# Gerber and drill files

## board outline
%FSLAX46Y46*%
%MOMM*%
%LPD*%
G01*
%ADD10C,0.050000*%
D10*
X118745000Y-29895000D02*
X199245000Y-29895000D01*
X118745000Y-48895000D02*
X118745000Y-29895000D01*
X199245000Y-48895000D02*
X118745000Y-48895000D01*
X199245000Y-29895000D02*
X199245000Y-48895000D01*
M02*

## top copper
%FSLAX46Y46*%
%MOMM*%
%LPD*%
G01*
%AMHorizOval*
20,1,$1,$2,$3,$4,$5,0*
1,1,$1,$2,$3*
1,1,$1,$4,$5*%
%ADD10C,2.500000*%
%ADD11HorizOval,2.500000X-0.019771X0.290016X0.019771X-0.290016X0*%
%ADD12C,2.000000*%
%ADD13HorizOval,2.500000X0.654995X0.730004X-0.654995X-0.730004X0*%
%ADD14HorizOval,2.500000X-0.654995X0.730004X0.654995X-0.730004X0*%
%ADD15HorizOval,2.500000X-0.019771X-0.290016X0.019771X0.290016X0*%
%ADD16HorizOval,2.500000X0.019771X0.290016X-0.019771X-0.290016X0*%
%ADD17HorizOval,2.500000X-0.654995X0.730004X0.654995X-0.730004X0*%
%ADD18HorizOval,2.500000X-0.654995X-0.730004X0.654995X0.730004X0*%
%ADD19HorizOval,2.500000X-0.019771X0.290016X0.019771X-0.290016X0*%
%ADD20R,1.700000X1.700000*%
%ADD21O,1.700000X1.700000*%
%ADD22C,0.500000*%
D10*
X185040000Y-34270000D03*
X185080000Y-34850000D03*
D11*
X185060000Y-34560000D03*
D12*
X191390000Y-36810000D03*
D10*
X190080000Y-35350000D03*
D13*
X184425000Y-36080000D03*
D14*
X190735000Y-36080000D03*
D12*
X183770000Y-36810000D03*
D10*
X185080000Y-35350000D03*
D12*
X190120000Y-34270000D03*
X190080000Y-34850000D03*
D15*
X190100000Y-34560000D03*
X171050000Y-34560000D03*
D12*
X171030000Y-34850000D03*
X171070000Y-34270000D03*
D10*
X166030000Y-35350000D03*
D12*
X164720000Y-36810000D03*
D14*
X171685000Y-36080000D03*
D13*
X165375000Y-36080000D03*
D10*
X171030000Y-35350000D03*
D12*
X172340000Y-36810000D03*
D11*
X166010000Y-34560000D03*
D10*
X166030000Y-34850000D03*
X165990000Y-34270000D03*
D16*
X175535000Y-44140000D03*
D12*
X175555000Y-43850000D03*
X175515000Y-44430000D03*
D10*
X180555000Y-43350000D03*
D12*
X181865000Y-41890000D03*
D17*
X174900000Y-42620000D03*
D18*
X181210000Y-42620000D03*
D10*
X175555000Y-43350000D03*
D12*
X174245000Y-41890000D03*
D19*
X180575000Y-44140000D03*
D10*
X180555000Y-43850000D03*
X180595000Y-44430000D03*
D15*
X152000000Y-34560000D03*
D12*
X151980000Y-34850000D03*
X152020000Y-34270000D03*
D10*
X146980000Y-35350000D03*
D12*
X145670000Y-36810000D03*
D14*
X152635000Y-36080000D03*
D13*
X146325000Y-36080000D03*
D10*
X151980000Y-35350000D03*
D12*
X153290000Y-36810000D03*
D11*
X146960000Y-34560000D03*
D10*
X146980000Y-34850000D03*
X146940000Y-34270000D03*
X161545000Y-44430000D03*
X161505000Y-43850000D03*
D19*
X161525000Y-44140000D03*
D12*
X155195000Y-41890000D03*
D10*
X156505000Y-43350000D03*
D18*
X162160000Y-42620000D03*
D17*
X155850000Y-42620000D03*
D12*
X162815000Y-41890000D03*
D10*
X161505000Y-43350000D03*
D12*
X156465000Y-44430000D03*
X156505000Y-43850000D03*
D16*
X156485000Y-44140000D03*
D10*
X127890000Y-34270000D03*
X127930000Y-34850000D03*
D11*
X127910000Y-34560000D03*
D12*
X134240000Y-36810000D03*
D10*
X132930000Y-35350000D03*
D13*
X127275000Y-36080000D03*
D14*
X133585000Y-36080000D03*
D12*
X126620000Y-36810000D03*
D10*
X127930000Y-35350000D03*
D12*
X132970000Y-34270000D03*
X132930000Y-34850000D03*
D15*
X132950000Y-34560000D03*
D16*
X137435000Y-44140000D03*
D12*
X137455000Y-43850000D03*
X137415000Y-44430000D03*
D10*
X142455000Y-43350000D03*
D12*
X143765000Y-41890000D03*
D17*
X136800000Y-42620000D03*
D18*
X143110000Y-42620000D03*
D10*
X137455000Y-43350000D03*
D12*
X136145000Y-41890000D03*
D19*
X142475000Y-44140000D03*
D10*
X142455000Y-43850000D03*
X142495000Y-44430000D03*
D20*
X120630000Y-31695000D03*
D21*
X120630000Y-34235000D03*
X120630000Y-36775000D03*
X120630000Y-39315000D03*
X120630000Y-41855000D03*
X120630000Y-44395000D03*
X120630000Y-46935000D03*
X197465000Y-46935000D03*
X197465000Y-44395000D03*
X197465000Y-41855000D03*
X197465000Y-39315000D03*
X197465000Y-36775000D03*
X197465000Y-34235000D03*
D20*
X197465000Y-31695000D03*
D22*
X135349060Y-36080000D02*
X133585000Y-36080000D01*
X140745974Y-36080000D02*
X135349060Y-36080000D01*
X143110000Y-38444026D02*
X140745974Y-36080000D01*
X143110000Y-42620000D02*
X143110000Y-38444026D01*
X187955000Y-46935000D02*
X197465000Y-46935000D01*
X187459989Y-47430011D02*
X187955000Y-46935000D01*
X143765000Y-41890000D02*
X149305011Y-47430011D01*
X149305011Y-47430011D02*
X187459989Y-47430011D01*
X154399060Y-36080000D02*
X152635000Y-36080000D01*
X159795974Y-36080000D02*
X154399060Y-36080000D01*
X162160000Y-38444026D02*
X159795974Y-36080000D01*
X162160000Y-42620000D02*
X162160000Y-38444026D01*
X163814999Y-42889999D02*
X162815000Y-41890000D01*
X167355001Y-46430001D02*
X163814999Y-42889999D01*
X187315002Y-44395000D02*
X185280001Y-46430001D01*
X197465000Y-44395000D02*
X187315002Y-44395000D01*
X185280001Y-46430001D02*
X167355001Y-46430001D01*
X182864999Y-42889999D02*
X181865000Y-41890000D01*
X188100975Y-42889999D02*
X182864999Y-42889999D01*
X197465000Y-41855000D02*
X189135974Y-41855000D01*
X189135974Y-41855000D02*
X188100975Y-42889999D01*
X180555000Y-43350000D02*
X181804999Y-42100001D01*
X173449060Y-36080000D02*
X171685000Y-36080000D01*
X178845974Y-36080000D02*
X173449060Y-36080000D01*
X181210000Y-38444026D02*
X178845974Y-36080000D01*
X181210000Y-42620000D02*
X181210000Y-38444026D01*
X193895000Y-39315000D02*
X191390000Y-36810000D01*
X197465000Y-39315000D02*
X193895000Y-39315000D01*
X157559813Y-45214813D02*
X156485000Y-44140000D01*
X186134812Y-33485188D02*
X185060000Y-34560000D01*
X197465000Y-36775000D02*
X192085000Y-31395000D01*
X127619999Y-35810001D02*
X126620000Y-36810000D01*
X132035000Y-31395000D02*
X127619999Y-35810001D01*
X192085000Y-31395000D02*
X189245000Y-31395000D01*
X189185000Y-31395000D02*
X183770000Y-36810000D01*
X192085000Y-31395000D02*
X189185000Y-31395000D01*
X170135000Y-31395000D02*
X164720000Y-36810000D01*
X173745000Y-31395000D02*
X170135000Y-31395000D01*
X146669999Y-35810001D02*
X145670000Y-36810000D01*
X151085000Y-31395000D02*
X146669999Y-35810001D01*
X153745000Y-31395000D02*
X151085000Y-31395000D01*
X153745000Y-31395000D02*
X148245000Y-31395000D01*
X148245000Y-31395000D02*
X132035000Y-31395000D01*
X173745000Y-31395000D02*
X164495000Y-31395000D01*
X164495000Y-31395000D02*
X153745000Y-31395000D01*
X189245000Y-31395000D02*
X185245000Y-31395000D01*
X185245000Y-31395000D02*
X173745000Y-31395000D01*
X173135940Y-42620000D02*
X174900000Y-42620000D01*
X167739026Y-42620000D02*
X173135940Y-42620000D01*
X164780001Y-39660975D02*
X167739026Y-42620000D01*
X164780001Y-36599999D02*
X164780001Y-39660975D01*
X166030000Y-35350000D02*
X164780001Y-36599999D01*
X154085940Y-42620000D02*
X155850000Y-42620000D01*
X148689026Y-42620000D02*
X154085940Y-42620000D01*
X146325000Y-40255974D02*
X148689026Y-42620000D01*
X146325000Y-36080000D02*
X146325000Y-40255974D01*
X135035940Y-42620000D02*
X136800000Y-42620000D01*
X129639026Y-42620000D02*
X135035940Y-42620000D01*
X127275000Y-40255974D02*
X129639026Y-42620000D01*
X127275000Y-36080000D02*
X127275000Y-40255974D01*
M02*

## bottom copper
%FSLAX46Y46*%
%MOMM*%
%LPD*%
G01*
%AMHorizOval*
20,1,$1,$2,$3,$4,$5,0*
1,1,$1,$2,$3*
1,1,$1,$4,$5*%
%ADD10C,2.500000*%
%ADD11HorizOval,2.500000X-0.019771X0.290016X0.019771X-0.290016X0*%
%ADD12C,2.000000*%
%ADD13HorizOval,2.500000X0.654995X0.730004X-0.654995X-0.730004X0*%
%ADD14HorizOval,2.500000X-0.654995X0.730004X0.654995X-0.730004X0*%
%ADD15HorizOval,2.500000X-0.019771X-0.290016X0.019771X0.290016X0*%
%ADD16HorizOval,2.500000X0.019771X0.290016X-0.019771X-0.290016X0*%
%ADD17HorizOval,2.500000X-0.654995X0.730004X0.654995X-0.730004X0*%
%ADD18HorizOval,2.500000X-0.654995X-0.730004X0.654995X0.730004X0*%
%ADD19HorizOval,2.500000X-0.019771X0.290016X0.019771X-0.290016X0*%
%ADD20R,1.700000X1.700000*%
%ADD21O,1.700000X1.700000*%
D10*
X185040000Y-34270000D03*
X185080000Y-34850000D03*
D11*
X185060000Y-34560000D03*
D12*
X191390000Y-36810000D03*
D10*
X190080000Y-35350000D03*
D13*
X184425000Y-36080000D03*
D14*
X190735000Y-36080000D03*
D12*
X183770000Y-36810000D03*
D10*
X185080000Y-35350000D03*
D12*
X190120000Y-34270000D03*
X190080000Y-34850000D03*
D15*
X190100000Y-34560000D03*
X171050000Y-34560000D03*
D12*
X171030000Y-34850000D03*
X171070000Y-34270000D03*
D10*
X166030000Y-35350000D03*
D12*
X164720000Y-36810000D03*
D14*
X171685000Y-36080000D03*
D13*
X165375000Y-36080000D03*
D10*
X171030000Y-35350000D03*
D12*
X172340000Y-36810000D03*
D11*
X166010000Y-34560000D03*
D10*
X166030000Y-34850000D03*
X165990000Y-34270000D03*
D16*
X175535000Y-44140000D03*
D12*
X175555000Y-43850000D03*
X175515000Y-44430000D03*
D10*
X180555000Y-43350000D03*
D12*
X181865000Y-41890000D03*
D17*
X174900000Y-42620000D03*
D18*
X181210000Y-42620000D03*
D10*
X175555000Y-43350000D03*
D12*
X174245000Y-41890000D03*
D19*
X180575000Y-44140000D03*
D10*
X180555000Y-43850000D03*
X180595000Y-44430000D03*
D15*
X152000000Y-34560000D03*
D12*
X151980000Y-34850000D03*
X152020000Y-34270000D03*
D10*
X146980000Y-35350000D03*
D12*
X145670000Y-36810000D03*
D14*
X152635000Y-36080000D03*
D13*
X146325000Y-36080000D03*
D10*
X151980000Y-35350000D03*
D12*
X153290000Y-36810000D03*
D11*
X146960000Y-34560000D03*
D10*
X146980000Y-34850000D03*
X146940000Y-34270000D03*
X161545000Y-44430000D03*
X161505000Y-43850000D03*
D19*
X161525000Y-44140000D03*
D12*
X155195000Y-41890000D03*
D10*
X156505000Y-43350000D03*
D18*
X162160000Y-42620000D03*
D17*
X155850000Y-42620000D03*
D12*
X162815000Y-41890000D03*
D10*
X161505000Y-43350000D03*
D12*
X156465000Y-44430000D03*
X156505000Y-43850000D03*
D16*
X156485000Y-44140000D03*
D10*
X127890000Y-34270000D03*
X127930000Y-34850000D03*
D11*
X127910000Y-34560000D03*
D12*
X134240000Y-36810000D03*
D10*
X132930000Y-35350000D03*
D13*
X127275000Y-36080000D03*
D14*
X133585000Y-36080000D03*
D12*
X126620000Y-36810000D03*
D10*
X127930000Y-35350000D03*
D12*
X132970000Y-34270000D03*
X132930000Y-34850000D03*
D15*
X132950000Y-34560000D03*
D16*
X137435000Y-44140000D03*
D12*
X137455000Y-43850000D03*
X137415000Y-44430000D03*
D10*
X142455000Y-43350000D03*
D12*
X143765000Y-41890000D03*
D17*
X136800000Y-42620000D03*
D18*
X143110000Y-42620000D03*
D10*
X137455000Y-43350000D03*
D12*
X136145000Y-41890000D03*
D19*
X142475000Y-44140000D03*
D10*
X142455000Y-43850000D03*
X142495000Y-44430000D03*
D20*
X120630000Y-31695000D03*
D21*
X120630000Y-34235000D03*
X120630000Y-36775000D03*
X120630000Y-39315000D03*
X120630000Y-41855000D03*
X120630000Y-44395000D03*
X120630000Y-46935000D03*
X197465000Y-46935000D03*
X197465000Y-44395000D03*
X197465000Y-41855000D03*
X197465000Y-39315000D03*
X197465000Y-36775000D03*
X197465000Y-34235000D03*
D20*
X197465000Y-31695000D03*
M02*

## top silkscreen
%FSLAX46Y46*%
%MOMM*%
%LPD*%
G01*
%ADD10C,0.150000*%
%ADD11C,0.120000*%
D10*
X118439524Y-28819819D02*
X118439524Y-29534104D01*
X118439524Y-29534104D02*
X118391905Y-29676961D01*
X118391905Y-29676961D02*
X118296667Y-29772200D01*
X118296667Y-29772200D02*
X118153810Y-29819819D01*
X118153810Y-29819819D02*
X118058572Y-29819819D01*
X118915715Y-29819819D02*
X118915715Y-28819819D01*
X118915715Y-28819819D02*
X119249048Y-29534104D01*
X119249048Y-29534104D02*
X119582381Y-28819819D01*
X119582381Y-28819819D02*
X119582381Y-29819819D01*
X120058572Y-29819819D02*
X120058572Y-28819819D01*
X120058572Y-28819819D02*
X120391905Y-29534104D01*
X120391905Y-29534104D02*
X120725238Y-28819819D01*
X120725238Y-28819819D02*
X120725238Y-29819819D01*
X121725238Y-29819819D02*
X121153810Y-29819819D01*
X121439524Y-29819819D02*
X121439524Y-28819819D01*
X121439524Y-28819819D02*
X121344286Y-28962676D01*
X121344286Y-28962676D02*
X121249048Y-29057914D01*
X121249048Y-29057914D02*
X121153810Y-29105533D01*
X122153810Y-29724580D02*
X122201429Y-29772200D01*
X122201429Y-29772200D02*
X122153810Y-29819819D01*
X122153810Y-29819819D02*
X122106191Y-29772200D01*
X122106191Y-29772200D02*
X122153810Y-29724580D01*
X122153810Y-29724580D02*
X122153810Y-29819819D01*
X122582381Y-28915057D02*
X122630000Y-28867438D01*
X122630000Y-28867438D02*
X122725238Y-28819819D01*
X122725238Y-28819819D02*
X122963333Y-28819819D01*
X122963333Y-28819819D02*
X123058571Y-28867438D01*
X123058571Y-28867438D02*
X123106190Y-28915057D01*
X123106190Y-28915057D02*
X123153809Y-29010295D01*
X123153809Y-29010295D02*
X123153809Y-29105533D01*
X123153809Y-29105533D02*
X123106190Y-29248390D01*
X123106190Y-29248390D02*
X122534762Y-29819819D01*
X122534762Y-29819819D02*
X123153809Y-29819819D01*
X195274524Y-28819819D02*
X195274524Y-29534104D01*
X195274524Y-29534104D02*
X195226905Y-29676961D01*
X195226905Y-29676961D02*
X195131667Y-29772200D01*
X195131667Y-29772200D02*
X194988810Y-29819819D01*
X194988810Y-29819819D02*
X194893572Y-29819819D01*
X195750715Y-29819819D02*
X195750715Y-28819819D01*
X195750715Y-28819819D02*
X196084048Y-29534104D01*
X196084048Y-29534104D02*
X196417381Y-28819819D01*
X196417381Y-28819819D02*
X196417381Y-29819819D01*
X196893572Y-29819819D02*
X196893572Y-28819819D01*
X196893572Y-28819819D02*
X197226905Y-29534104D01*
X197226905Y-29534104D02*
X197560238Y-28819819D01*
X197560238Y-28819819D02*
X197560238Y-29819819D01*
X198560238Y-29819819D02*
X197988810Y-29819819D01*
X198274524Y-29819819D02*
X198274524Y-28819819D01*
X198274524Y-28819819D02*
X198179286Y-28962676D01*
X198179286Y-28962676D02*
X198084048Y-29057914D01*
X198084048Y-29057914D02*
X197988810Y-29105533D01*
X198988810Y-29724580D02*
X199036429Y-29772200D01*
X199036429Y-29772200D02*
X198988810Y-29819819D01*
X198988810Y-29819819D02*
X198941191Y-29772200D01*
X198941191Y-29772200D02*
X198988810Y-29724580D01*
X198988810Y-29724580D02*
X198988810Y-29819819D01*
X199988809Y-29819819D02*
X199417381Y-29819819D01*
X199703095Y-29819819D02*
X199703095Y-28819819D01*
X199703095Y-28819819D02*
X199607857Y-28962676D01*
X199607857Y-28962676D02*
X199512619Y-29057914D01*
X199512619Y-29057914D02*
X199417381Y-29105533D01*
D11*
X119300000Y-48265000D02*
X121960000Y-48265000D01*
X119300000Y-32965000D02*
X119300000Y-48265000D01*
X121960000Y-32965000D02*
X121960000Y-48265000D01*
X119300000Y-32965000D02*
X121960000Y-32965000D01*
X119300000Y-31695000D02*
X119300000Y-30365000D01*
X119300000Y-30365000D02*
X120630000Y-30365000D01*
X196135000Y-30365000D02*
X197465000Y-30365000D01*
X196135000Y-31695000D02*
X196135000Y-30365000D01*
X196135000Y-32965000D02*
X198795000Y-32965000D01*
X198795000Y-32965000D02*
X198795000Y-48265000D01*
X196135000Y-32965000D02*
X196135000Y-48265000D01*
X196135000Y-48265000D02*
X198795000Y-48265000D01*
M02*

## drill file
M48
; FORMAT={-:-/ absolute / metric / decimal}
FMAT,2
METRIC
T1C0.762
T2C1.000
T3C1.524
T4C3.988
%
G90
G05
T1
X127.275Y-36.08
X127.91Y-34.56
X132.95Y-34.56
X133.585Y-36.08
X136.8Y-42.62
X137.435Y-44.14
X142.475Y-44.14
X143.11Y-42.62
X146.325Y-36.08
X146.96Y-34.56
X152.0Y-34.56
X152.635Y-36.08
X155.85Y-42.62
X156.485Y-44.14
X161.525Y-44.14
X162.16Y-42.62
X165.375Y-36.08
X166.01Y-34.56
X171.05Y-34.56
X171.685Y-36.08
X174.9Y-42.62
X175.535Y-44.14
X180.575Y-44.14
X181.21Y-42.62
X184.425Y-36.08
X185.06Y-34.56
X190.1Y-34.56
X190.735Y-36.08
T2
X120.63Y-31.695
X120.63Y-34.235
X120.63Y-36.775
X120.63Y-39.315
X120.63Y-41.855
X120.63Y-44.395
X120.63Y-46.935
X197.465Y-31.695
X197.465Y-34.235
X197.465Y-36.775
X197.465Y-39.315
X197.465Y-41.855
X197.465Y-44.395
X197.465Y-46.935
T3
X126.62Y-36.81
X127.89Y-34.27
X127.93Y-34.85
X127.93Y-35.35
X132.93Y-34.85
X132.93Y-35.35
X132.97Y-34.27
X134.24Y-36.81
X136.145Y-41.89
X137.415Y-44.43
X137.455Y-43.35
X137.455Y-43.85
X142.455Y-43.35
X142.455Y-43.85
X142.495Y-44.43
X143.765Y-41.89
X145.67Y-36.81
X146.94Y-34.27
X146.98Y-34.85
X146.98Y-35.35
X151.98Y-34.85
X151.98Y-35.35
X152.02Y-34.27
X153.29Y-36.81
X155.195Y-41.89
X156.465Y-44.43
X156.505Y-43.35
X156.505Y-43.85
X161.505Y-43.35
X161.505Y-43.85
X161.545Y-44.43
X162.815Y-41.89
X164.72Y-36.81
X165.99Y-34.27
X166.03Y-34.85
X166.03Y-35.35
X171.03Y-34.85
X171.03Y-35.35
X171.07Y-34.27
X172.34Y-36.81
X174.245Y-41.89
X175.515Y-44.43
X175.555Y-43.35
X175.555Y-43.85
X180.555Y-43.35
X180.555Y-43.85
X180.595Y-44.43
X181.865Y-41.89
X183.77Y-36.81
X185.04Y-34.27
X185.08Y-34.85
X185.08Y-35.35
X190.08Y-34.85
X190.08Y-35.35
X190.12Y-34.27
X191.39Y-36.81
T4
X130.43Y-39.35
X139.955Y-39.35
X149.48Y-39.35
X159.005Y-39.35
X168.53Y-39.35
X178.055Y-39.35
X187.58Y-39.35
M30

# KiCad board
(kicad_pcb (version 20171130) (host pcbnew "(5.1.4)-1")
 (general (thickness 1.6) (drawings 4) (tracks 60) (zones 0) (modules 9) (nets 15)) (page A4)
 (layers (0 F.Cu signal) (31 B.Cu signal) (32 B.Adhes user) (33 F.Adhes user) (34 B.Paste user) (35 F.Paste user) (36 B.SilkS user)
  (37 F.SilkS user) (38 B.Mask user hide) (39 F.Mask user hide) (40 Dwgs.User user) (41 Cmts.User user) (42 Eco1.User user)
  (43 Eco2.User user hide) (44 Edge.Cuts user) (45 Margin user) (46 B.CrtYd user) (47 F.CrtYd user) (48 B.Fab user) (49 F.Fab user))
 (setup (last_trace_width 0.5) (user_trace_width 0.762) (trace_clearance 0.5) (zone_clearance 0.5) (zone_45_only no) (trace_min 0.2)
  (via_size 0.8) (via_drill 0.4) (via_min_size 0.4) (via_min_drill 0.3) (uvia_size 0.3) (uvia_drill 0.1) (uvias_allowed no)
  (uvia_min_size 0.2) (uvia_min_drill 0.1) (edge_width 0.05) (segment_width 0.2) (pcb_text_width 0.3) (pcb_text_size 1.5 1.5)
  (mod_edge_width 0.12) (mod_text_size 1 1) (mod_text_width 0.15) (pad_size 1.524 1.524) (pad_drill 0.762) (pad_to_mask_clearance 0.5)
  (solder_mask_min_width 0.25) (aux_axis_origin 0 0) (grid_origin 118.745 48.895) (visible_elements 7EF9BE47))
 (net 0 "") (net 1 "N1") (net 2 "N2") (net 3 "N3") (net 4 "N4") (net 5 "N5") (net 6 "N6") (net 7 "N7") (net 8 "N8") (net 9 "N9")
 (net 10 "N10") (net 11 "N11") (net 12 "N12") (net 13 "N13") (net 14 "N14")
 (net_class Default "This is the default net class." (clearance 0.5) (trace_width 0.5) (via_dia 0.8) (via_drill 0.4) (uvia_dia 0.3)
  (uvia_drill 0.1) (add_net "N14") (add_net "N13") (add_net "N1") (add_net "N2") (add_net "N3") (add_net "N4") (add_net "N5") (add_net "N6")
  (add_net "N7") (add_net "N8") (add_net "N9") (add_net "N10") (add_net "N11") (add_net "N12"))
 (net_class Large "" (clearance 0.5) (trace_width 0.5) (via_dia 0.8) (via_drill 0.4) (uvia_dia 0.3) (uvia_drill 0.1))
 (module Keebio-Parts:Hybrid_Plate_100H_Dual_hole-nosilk (layer F.Cu) (at 187.58 39.35)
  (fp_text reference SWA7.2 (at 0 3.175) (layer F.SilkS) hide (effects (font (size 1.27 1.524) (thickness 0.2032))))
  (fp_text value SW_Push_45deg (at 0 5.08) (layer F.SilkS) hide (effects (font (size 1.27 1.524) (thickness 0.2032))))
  (pad 1 thru_hole circle (at -2.54 -5.08 330.9) (size 2.5 2.5) (drill 1.524) (layers *.Cu F.Mask) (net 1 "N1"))
  (pad 1 thru_hole circle (at -2.5 -4.5 330.9) (size 2.5 2.5) (drill 1.524) (layers *.Cu F.Mask) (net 1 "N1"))
  (pad 1 thru_hole oval (at -2.52 -4.79 3.9) (size 2.5 3.081378) (drill 0.762) (layers *.Cu F.Mask) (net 1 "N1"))
  (pad 2 thru_hole circle (at 3.81 -2.54 330.9) (size 2 2) (drill 1.524) (layers *.Cu F.Mask) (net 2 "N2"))
  (pad 2 thru_hole circle (at 2.5 -4) (size 2.5 2.5) (drill 1.524) (layers *.Cu *.Mask) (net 2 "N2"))
  (pad 1 thru_hole oval (at -3.155 -3.27 138.1) (size 2.5 4.461556) (drill 0.762) (layers *.Cu B.Mask) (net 1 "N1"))
  (pad 2 thru_hole oval (at 3.155 -3.27 221.9) (size 2.5 4.461556) (drill 0.762) (layers *.Cu F.Mask) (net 2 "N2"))
  (pad 1 thru_hole circle (at -3.81 -2.54 330.9) (size 2 2) (drill 1.524) (layers *.Cu B.Mask) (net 1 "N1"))
  (pad HOLE np_thru_hole circle (at 0 0) (size 3.9878 3.9878) (drill 3.9878) (layers *.Cu *.Mask))
  (pad 1 thru_hole circle (at -2.5 -4 330.9) (size 2.5 2.5) (drill 1.524) (layers *.Cu *.Mask) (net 1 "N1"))
  (pad 2 thru_hole circle (at 2.54 -5.08 330.9) (size 2 2) (drill 1.524) (layers *.Cu B.Mask) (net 2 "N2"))
  (pad 2 thru_hole circle (at 2.5 -4.5 330.9) (size 2 2) (drill 1.524) (layers *.Cu B.Mask) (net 2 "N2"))
  (pad 2 thru_hole oval (at 2.52 -4.79 356.1) (size 2.5 3.081378) (drill 0.762) (layers *.Cu B.Mask) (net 2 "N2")))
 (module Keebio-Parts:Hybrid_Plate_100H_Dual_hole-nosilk (layer F.Cu) (at 168.53 39.35)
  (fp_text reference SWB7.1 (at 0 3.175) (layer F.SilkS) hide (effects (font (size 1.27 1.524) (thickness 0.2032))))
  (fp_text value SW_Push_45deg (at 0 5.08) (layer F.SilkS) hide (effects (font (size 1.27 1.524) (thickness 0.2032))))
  (pad 2 thru_hole oval (at 2.52 -4.79 356.1) (size 2.5 3.081378) (drill 0.762) (layers *.Cu B.Mask) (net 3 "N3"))
  (pad 2 thru_hole circle (at 2.5 -4.5 330.9) (size 2 2) (drill 1.524) (layers *.Cu B.Mask) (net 3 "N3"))
  (pad 2 thru_hole circle (at 2.54 -5.08 330.9) (size 2 2) (drill 1.524) (layers *.Cu B.Mask) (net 3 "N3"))
  (pad 1 thru_hole circle (at -2.5 -4 330.9) (size 2.5 2.5) (drill 1.524) (layers *.Cu *.Mask) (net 1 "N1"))
  (pad HOLE np_thru_hole circle (at 0 0) (size 3.9878 3.9878) (drill 3.9878) (layers *.Cu *.Mask))
  (pad 1 thru_hole circle (at -3.81 -2.54 330.9) (size 2 2) (drill 1.524) (layers *.Cu B.Mask) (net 1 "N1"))
  (pad 2 thru_hole oval (at 3.155 -3.27 221.9) (size 2.5 4.461556) (drill 0.762) (layers *.Cu F.Mask) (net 3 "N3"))
  (pad 1 thru_hole oval (at -3.155 -3.27 138.1) (size 2.5 4.461556) (drill 0.762) (layers *.Cu B.Mask) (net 1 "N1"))
  (pad 2 thru_hole circle (at 2.5 -4) (size 2.5 2.5) (drill 1.524) (layers *.Cu *.Mask) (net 3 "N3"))
  (pad 2 thru_hole circle (at 3.81 -2.54 330.9) (size 2 2) (drill 1.524) (layers *.Cu F.Mask) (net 3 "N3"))
  (pad 1 thru_hole oval (at -2.52 -4.79 3.9) (size 2.5 3.081378) (drill 0.762) (layers *.Cu F.Mask) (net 1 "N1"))
  (pad 1 thru_hole circle (at -2.5 -4.5 330.9) (size 2.5 2.5) (drill 1.524) (layers *.Cu F.Mask) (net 1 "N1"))
  (pad 1 thru_hole circle (at -2.54 -5.08 330.9) (size 2.5 2.5) (drill 1.524) (layers *.Cu F.Mask) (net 1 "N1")))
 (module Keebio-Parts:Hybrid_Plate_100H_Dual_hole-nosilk (layer F.Cu) (at 178.055 39.35 180)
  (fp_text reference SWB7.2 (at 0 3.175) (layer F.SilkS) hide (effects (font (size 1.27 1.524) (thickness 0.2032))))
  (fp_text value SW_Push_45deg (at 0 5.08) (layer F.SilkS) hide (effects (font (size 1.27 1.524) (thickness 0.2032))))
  (pad 2 thru_hole oval (at 2.52 -4.79 176.1) (size 2.5 3.081378) (drill 0.762) (layers *.Cu B.Mask) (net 1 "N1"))
  (pad 2 thru_hole circle (at 2.5 -4.5 150.9) (size 2 2) (drill 1.524) (layers *.Cu B.Mask) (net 1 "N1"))
  (pad 2 thru_hole circle (at 2.54 -5.08 150.9) (size 2 2) (drill 1.524) (layers *.Cu B.Mask) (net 1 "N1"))
  (pad 1 thru_hole circle (at -2.5 -4 150.9) (size 2.5 2.5) (drill 1.524) (layers *.Cu *.Mask) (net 3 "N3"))
  (pad HOLE np_thru_hole circle (at 0 0 180) (size 3.9878 3.9878) (drill 3.9878) (layers *.Cu *.Mask))
  (pad 1 thru_hole circle (at -3.81 -2.54 150.9) (size 2 2) (drill 1.524) (layers *.Cu B.Mask) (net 3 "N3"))
  (pad 2 thru_hole oval (at 3.155 -3.27 41.9) (size 2.5 4.461556) (drill 0.762) (layers *.Cu F.Mask) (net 1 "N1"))
  (pad 1 thru_hole oval (at -3.155 -3.27 318.1) (size 2.5 4.461556) (drill 0.762) (layers *.Cu B.Mask) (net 3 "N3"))
  (pad 2 thru_hole circle (at 2.5 -4 180) (size 2.5 2.5) (drill 1.524) (layers *.Cu *.Mask) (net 1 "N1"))
  (pad 2 thru_hole circle (at 3.81 -2.54 150.9) (size 2 2) (drill 1.524) (layers *.Cu F.Mask) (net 1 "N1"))
  (pad 1 thru_hole oval (at -2.52 -4.79 183.9) (size 2.5 3.081378) (drill 0.762) (layers *.Cu F.Mask) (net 3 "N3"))
  (pad 1 thru_hole circle (at -2.5 -4.5 150.9) (size 2.5 2.5) (drill 1.524) (layers *.Cu F.Mask) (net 3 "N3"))
  (pad 1 thru_hole circle (at -2.54 -5.08 150.9) (size 2.5 2.5) (drill 1.524) (layers *.Cu F.Mask) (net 3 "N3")))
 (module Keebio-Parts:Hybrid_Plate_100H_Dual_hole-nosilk (layer F.Cu) (at 149.48 39.35)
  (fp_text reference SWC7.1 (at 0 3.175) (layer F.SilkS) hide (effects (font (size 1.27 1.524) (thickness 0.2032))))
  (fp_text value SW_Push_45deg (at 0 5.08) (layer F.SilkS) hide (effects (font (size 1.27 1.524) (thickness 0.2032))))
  (pad 2 thru_hole oval (at 2.52 -4.79 356.1) (size 2.5 3.081378) (drill 0.762) (layers *.Cu B.Mask) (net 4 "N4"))
  (pad 2 thru_hole circle (at 2.5 -4.5 330.9) (size 2 2) (drill 1.524) (layers *.Cu B.Mask) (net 4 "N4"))
  (pad 2 thru_hole circle (at 2.54 -5.08 330.9) (size 2 2) (drill 1.524) (layers *.Cu B.Mask) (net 4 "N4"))
  (pad 1 thru_hole circle (at -2.5 -4 330.9) (size 2.5 2.5) (drill 1.524) (layers *.Cu *.Mask) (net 1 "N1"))
  (pad HOLE np_thru_hole circle (at 0 0) (size 3.9878 3.9878) (drill 3.9878) (layers *.Cu *.Mask))
  (pad 1 thru_hole circle (at -3.81 -2.54 330.9) (size 2 2) (drill 1.524) (layers *.Cu B.Mask) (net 1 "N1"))
  (pad 2 thru_hole oval (at 3.155 -3.27 221.9) (size 2.5 4.461556) (drill 0.762) (layers *.Cu F.Mask) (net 4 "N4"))
  (pad 1 thru_hole oval (at -3.155 -3.27 138.1) (size 2.5 4.461556) (drill 0.762) (layers *.Cu B.Mask) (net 1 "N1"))
  (pad 2 thru_hole circle (at 2.5 -4) (size 2.5 2.5) (drill 1.524) (layers *.Cu *.Mask) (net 4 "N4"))
  (pad 2 thru_hole circle (at 3.81 -2.54 330.9) (size 2 2) (drill 1.524) (layers *.Cu F.Mask) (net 4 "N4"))
  (pad 1 thru_hole oval (at -2.52 -4.79 3.9) (size 2.5 3.081378) (drill 0.762) (layers *.Cu F.Mask) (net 1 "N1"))
  (pad 1 thru_hole circle (at -2.5 -4.5 330.9) (size 2.5 2.5) (drill 1.524) (layers *.Cu F.Mask) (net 1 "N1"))
  (pad 1 thru_hole circle (at -2.54 -5.08 330.9) (size 2.5 2.5) (drill 1.524) (layers *.Cu F.Mask) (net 1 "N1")))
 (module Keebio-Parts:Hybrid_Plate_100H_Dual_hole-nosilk (layer F.Cu) (at 159.005 39.35 180)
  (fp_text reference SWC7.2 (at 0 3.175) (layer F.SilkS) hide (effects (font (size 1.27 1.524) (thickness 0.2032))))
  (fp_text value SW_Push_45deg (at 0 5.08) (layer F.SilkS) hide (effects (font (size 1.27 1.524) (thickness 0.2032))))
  (pad 1 thru_hole circle (at -2.54 -5.08 150.9) (size 2.5 2.5) (drill 1.524) (layers *.Cu F.Mask) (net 4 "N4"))
  (pad 1 thru_hole circle (at -2.5 -4.5 150.9) (size 2.5 2.5) (drill 1.524) (layers *.Cu F.Mask) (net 4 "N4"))
  (pad 1 thru_hole oval (at -2.52 -4.79 183.9) (size 2.5 3.081378) (drill 0.762) (layers *.Cu F.Mask) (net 4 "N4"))
  (pad 2 thru_hole circle (at 3.81 -2.54 150.9) (size 2 2) (drill 1.524) (layers *.Cu F.Mask) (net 1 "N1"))
  (pad 2 thru_hole circle (at 2.5 -4 180) (size 2.5 2.5) (drill 1.524) (layers *.Cu *.Mask) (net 1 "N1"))
  (pad 1 thru_hole oval (at -3.155 -3.27 318.1) (size 2.5 4.461556) (drill 0.762) (layers *.Cu B.Mask) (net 4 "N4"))
  (pad 2 thru_hole oval (at 3.155 -3.27 41.9) (size 2.5 4.461556) (drill 0.762) (layers *.Cu F.Mask) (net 1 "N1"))
  (pad 1 thru_hole circle (at -3.81 -2.54 150.9) (size 2 2) (drill 1.524) (layers *.Cu B.Mask) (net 4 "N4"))
  (pad HOLE np_thru_hole circle (at 0 0 180) (size 3.9878 3.9878) (drill 3.9878) (layers *.Cu *.Mask))
  (pad 1 thru_hole circle (at -2.5 -4 150.9) (size 2.5 2.5) (drill 1.524) (layers *.Cu *.Mask) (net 4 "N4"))
  (pad 2 thru_hole circle (at 2.54 -5.08 150.9) (size 2 2) (drill 1.524) (layers *.Cu B.Mask) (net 1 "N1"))
  (pad 2 thru_hole circle (at 2.5 -4.5 150.9) (size 2 2) (drill 1.524) (layers *.Cu B.Mask) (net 1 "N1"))
  (pad 2 thru_hole oval (at 2.52 -4.79 176.1) (size 2.5 3.081378) (drill 0.762) (layers *.Cu B.Mask) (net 1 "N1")))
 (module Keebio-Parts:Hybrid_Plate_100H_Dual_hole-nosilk (layer F.Cu) (at 130.43 39.35)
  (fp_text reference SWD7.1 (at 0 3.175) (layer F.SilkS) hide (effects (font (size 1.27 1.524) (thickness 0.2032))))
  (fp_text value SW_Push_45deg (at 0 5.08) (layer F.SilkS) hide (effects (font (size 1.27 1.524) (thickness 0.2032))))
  (pad 1 thru_hole circle (at -2.54 -5.08 330.9) (size 2.5 2.5) (drill 1.524) (layers *.Cu F.Mask) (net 1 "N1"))
  (pad 1 thru_hole circle (at -2.5 -4.5 330.9) (size 2.5 2.5) (drill 1.524) (layers *.Cu F.Mask) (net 1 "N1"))
  (pad 1 thru_hole oval (at -2.52 -4.79 3.9) (size 2.5 3.081378) (drill 0.762) (layers *.Cu F.Mask) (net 1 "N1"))
  (pad 2 thru_hole circle (at 3.81 -2.54 330.9) (size 2 2) (drill 1.524) (layers *.Cu F.Mask) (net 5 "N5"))
  (pad 2 thru_hole circle (at 2.5 -4) (size 2.5 2.5) (drill 1.524) (layers *.Cu *.Mask) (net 5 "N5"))
  (pad 1 thru_hole oval (at -3.155 -3.27 138.1) (size 2.5 4.461556) (drill 0.762) (layers *.Cu B.Mask) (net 1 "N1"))
  (pad 2 thru_hole oval (at 3.155 -3.27 221.9) (size 2.5 4.461556) (drill 0.762) (layers *.Cu F.Mask) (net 5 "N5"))
  (pad 1 thru_hole circle (at -3.81 -2.54 330.9) (size 2 2) (drill 1.524) (layers *.Cu B.Mask) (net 1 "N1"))
  (pad HOLE np_thru_hole circle (at 0 0) (size 3.9878 3.9878) (drill 3.9878) (layers *.Cu *.Mask))
  (pad 1 thru_hole circle (at -2.5 -4 330.9) (size 2.5 2.5) (drill 1.524) (layers *.Cu *.Mask) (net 1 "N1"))
  (pad 2 thru_hole circle (at 2.54 -5.08 330.9) (size 2 2) (drill 1.524) (layers *.Cu B.Mask) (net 5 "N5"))
  (pad 2 thru_hole circle (at 2.5 -4.5 330.9) (size 2 2) (drill 1.524) (layers *.Cu B.Mask) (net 5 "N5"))
  (pad 2 thru_hole oval (at 2.52 -4.79 356.1) (size 2.5 3.081378) (drill 0.762) (layers *.Cu B.Mask) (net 5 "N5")))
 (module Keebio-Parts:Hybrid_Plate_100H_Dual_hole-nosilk (layer F.Cu) (at 139.955 39.35 180)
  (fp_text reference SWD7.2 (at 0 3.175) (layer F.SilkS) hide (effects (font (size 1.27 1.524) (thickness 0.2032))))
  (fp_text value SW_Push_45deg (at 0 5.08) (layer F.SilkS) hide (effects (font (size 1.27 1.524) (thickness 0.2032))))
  (pad 2 thru_hole oval (at 2.52 -4.79 176.1) (size 2.5 3.081378) (drill 0.762) (layers *.Cu B.Mask) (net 1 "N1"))
  (pad 2 thru_hole circle (at 2.5 -4.5 150.9) (size 2 2) (drill 1.524) (layers *.Cu B.Mask) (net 1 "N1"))
  (pad 2 thru_hole circle (at 2.54 -5.08 150.9) (size 2 2) (drill 1.524) (layers *.Cu B.Mask) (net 1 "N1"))
  (pad 1 thru_hole circle (at -2.5 -4 150.9) (size 2.5 2.5) (drill 1.524) (layers *.Cu *.Mask) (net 5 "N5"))
  (pad HOLE np_thru_hole circle (at 0 0 180) (size 3.9878 3.9878) (drill 3.9878) (layers *.Cu *.Mask))
  (pad 1 thru_hole circle (at -3.81 -2.54 150.9) (size 2 2) (drill 1.524) (layers *.Cu B.Mask) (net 5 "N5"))
  (pad 2 thru_hole oval (at 3.155 -3.27 41.9) (size 2.5 4.461556) (drill 0.762) (layers *.Cu F.Mask) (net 1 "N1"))
  (pad 1 thru_hole oval (at -3.155 -3.27 318.1) (size 2.5 4.461556) (drill 0.762) (layers *.Cu B.Mask) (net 5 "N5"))
  (pad 2 thru_hole circle (at 2.5 -4 180) (size 2.5 2.5) (drill 1.524) (layers *.Cu *.Mask) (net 1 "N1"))
  (pad 2 thru_hole circle (at 3.81 -2.54 150.9) (size 2 2) (drill 1.524) (layers *.Cu F.Mask) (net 1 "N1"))
  (pad 1 thru_hole oval (at -2.52 -4.79 183.9) (size 2.5 3.081378) (drill 0.762) (layers *.Cu F.Mask) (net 5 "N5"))
  (pad 1 thru_hole circle (at -2.5 -4.5 150.9) (size 2.5 2.5) (drill 1.524) (layers *.Cu F.Mask) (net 5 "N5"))
  (pad 1 thru_hole circle (at -2.54 -5.08 150.9) (size 2.5 2.5) (drill 1.524) (layers *.Cu F.Mask) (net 5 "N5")))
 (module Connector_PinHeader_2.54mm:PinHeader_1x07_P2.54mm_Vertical (layer F.Cu) (at 120.63 31.695)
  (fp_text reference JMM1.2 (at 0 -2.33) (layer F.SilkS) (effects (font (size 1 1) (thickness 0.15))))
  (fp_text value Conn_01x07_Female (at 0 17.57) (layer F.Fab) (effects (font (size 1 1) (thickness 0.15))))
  (fp_line (start -1.33 16.57) (end 1.33 16.57) (layer F.SilkS) (width 0.12))
  (fp_line (start -1.33 1.27) (end -1.33 16.57) (layer F.SilkS) (width 0.12))
  (fp_line (start 1.33 1.27) (end 1.33 16.57) (layer F.SilkS) (width 0.12))
  (fp_line (start -1.33 1.27) (end 1.33 1.27) (layer F.SilkS) (width 0.12))
  (fp_line (start -1.33 0) (end -1.33 -1.33) (layer F.SilkS) (width 0.12))
  (fp_line (start -1.33 -1.33) (end 0 -1.33) (layer F.SilkS) (width 0.12))
  (pad 1 thru_hole rect (at 0 0) (size 1.7 1.7) (drill 1) (layers *.Cu *.Mask) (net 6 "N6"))
  (pad 2 thru_hole oval (at 0 2.54) (size 1.7 1.7) (drill 1) (layers *.Cu *.Mask) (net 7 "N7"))
  (pad 3 thru_hole oval (at 0 5.08) (size 1.7 1.7) (drill 1) (layers *.Cu *.Mask) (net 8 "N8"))
  (pad 4 thru_hole oval (at 0 7.62) (size 1.7 1.7) (drill 1) (layers *.Cu *.Mask) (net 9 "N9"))
  (pad 5 thru_hole oval (at 0 10.16) (size 1.7 1.7) (drill 1) (layers *.Cu *.Mask) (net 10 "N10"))
  (pad 6 thru_hole oval (at 0 12.7) (size 1.7 1.7) (drill 1) (layers *.Cu *.Mask) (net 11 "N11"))
  (pad 7 thru_hole oval (at 0 15.24) (size 1.7 1.7) (drill 1) (layers *.Cu *.Mask) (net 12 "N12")))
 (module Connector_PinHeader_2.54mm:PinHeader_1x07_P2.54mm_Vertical (layer F.Cu) (at 197.465 31.695)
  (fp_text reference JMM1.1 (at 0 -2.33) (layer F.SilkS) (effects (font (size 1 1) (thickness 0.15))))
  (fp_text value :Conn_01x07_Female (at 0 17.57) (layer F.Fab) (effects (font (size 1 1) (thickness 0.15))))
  (fp_line (start -1.33 -1.33) (end 0 -1.33) (layer F.SilkS) (width 0.12))
  (fp_line (start -1.33 0) (end -1.33 -1.33) (layer F.SilkS) (width 0.12))
  (fp_line (start -1.33 1.27) (end 1.33 1.27) (layer F.SilkS) (width 0.12))
  (fp_line (start 1.33 1.27) (end 1.33 16.57) (layer F.SilkS) (width 0.12))
  (fp_line (start -1.33 1.27) (end -1.33 16.57) (layer F.SilkS) (width 0.12))
  (fp_line (start -1.33 16.57) (end 1.33 16.57) (layer F.SilkS) (width 0.12))
  (pad 7 thru_hole oval (at 0 15.24) (size 1.7 1.7) (drill 1) (layers *.Cu *.Mask) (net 5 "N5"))
  (pad 6 thru_hole oval (at 0 12.7) (size 1.7 1.7) (drill 1) (layers *.Cu *.Mask) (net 4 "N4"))
  (pad 5 thru_hole oval (at 0 10.16) (size 1.7 1.7) (drill 1) (layers *.Cu *.Mask) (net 3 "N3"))
  (pad 4 thru_hole oval (at 0 7.62) (size 1.7 1.7) (drill 1) (layers *.Cu *.Mask) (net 2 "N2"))
  (pad 3 thru_hole oval (at 0 5.08) (size 1.7 1.7) (drill 1) (layers *.Cu *.Mask) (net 1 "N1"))
  (pad 2 thru_hole oval (at 0 2.54) (size 1.7 1.7) (drill 1) (layers *.Cu *.Mask) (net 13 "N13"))
  (pad 1 thru_hole rect (at 0 0) (size 1.7 1.7) (drill 1) (layers *.Cu *.Mask) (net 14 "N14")))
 (gr_line (start 118.745 29.895) (end 199.245 29.895) (layer Edge.Cuts) (width 0.05))
 (gr_line (start 118.745 48.895) (end 118.745 29.895) (layer Edge.Cuts) (width 0.05))
 (gr_line (start 199.245 48.895) (end 118.745 48.895) (layer Edge.Cuts) (width 0.05))
 (gr_line (start 199.245 29.895) (end 199.245 48.895) (layer Edge.Cuts) (width 0.05))
 (segment (start 135.34906 36.08) (end 133.585 36.08) (width 0.5) (layer F.Cu) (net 5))
 (segment (start 140.745974 36.08) (end 135.34906 36.08) (width 0.5) (layer F.Cu) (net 5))
 (segment (start 143.11 38.444026) (end 140.745974 36.08) (width 0.5) (layer F.Cu) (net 5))
 (segment (start 143.11 42.62) (end 143.11 38.444026) (width 0.5) (layer F.Cu) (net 5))
 (segment (start 187.955 46.935) (end 197.465 46.935) (width 0.5) (layer F.Cu) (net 5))
 (segment (start 187.459989 47.430011) (end 187.955 46.935) (width 0.5) (layer F.Cu) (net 5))
 (segment (start 143.765 41.89) (end 149.305011 47.430011) (width 0.5) (layer F.Cu) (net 5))
 (segment (start 149.305011 47.430011) (end 187.459989 47.430011) (width 0.5) (layer F.Cu) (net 5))
 (segment (start 154.39906 36.08) (end 152.635 36.08) (width 0.5) (layer F.Cu) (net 4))
 (segment (start 159.795974 36.08) (end 154.39906 36.08) (width 0.5) (layer F.Cu) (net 4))
 (segment (start 162.16 38.444026) (end 159.795974 36.08) (width 0.5) (layer F.Cu) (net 4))
 (segment (start 162.16 42.62) (end 162.16 38.444026) (width 0.5) (layer F.Cu) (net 4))
 (segment (start 163.814999 42.889999) (end 162.815 41.89) (width 0.5) (layer F.Cu) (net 4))
 (segment (start 167.355001 46.430001) (end 163.814999 42.889999) (width 0.5) (layer F.Cu) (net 4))
 (segment (start 187.315002 44.395) (end 185.280001 46.430001) (width 0.5) (layer F.Cu) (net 4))
 (segment (start 197.465 44.395) (end 187.315002 44.395) (width 0.5) (layer F.Cu) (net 4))
 (segment (start 185.280001 46.430001) (end 167.355001 46.430001) (width 0.5) (layer F.Cu) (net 4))
 (segment (start 182.864999 42.889999) (end 181.865 41.89) (width 0.5) (layer F.Cu) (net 3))
 (segment (start 188.100975 42.889999) (end 182.864999 42.889999) (width 0.5) (layer F.Cu) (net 3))
 (segment (start 197.465 41.855) (end 189.135974 41.855) (width 0.5) (layer F.Cu) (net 3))
 (segment (start 189.135974 41.855) (end 188.100975 42.889999) (width 0.5) (layer F.Cu) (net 3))
 (segment (start 180.555 43.35) (end 181.804999 42.100001) (width 0.5) (layer F.Cu) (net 3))
 (segment (start 173.44906 36.08) (end 171.685 36.08) (width 0.5) (layer F.Cu) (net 3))
 (segment (start 178.845974 36.08) (end 173.44906 36.08) (width 0.5) (layer F.Cu) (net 3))
 (segment (start 181.21 38.444026) (end 178.845974 36.08) (width 0.5) (layer F.Cu) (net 3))
 (segment (start 181.21 42.62) (end 181.21 38.444026) (width 0.5) (layer F.Cu) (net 3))
 (segment (start 193.895 39.315) (end 191.39 36.81) (width 0.5) (layer F.Cu) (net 2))
 (segment (start 197.465 39.315) (end 193.895 39.315) (width 0.5) (layer F.Cu) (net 2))
 (segment (start 157.559813 45.214813) (end 156.485 44.14) (width 0.5) (layer F.Cu) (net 1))
 (segment (start 186.134812 33.485188) (end 185.06 34.56) (width 0.5) (layer F.Cu) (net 1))
 (segment (start 197.465 36.775) (end 192.085 31.395) (width 0.5) (layer F.Cu) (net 1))
 (segment (start 127.619999 35.810001) (end 126.62 36.81) (width 0.5) (layer F.Cu) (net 1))
 (segment (start 132.035 31.395) (end 127.619999 35.810001) (width 0.5) (layer F.Cu) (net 1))
 (segment (start 192.085 31.395) (end 189.245 31.395) (width 0.5) (layer F.Cu) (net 1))
 (segment (start 189.185 31.395) (end 183.77 36.81) (width 0.5) (layer F.Cu) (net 1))
 (segment (start 192.085 31.395) (end 189.185 31.395) (width 0.5) (layer F.Cu) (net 1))
 (segment (start 170.135 31.395) (end 164.72 36.81) (width 0.5) (layer F.Cu) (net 1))
 (segment (start 173.745 31.395) (end 170.135 31.395) (width 0.5) (layer F.Cu) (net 1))
 (segment (start 146.669999 35.810001) (end 145.67 36.81) (width 0.5) (layer F.Cu) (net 1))
 (segment (start 151.085 31.395) (end 146.669999 35.810001) (width 0.5) (layer F.Cu) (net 1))
 (segment (start 153.745 31.395) (end 151.085 31.395) (width 0.5) (layer F.Cu) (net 1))
 (segment (start 153.745 31.395) (end 148.245 31.395) (width 0.5) (layer F.Cu) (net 1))
 (segment (start 148.245 31.395) (end 132.035 31.395) (width 0.5) (layer F.Cu) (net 1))
 (segment (start 173.745 31.395) (end 164.495 31.395) (width 0.5) (layer F.Cu) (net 1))
 (segment (start 164.495 31.395) (end 153.745 31.395) (width 0.5) (layer F.Cu) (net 1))
 (segment (start 189.245 31.395) (end 185.245 31.395) (width 0.5) (layer F.Cu) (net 1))
 (segment (start 185.245 31.395) (end 173.745 31.395) (width 0.5) (layer F.Cu) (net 1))
 (segment (start 173.13594 42.62) (end 174.9 42.62) (width 0.5) (layer F.Cu) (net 1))
 (segment (start 167.739026 42.62) (end 173.13594 42.62) (width 0.5) (layer F.Cu) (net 1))
 (segment (start 164.780001 39.660975) (end 167.739026 42.62) (width 0.5) (layer F.Cu) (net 1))
 (segment (start 164.780001 36.599999) (end 164.780001 39.660975) (width 0.5) (layer F.Cu) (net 1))
 (segment (start 166.03 35.35) (end 164.780001 36.599999) (width 0.5) (layer F.Cu) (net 1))
 (segment (start 154.08594 42.62) (end 155.85 42.62) (width 0.5) (layer F.Cu) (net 1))
 (segment (start 148.689026 42.62) (end 154.08594 42.62) (width 0.5) (layer F.Cu) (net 1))
 (segment (start 146.325 40.255974) (end 148.689026 42.62) (width 0.5) (layer F.Cu) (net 1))
 (segment (start 146.325 36.08) (end 146.325 40.255974) (width 0.5) (layer F.Cu) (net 1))
 (segment (start 135.03594 42.62) (end 136.8 42.62) (width 0.5) (layer F.Cu) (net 1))
 (segment (start 129.639026 42.62) (end 135.03594 42.62) (width 0.5) (layer F.Cu) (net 1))
 (segment (start 127.275 40.255974) (end 129.639026 42.62) (width 0.5) (layer F.Cu) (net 1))
 (segment (start 127.275 36.08) (end 127.275 40.255974) (width 0.5) (layer F.Cu) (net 1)))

